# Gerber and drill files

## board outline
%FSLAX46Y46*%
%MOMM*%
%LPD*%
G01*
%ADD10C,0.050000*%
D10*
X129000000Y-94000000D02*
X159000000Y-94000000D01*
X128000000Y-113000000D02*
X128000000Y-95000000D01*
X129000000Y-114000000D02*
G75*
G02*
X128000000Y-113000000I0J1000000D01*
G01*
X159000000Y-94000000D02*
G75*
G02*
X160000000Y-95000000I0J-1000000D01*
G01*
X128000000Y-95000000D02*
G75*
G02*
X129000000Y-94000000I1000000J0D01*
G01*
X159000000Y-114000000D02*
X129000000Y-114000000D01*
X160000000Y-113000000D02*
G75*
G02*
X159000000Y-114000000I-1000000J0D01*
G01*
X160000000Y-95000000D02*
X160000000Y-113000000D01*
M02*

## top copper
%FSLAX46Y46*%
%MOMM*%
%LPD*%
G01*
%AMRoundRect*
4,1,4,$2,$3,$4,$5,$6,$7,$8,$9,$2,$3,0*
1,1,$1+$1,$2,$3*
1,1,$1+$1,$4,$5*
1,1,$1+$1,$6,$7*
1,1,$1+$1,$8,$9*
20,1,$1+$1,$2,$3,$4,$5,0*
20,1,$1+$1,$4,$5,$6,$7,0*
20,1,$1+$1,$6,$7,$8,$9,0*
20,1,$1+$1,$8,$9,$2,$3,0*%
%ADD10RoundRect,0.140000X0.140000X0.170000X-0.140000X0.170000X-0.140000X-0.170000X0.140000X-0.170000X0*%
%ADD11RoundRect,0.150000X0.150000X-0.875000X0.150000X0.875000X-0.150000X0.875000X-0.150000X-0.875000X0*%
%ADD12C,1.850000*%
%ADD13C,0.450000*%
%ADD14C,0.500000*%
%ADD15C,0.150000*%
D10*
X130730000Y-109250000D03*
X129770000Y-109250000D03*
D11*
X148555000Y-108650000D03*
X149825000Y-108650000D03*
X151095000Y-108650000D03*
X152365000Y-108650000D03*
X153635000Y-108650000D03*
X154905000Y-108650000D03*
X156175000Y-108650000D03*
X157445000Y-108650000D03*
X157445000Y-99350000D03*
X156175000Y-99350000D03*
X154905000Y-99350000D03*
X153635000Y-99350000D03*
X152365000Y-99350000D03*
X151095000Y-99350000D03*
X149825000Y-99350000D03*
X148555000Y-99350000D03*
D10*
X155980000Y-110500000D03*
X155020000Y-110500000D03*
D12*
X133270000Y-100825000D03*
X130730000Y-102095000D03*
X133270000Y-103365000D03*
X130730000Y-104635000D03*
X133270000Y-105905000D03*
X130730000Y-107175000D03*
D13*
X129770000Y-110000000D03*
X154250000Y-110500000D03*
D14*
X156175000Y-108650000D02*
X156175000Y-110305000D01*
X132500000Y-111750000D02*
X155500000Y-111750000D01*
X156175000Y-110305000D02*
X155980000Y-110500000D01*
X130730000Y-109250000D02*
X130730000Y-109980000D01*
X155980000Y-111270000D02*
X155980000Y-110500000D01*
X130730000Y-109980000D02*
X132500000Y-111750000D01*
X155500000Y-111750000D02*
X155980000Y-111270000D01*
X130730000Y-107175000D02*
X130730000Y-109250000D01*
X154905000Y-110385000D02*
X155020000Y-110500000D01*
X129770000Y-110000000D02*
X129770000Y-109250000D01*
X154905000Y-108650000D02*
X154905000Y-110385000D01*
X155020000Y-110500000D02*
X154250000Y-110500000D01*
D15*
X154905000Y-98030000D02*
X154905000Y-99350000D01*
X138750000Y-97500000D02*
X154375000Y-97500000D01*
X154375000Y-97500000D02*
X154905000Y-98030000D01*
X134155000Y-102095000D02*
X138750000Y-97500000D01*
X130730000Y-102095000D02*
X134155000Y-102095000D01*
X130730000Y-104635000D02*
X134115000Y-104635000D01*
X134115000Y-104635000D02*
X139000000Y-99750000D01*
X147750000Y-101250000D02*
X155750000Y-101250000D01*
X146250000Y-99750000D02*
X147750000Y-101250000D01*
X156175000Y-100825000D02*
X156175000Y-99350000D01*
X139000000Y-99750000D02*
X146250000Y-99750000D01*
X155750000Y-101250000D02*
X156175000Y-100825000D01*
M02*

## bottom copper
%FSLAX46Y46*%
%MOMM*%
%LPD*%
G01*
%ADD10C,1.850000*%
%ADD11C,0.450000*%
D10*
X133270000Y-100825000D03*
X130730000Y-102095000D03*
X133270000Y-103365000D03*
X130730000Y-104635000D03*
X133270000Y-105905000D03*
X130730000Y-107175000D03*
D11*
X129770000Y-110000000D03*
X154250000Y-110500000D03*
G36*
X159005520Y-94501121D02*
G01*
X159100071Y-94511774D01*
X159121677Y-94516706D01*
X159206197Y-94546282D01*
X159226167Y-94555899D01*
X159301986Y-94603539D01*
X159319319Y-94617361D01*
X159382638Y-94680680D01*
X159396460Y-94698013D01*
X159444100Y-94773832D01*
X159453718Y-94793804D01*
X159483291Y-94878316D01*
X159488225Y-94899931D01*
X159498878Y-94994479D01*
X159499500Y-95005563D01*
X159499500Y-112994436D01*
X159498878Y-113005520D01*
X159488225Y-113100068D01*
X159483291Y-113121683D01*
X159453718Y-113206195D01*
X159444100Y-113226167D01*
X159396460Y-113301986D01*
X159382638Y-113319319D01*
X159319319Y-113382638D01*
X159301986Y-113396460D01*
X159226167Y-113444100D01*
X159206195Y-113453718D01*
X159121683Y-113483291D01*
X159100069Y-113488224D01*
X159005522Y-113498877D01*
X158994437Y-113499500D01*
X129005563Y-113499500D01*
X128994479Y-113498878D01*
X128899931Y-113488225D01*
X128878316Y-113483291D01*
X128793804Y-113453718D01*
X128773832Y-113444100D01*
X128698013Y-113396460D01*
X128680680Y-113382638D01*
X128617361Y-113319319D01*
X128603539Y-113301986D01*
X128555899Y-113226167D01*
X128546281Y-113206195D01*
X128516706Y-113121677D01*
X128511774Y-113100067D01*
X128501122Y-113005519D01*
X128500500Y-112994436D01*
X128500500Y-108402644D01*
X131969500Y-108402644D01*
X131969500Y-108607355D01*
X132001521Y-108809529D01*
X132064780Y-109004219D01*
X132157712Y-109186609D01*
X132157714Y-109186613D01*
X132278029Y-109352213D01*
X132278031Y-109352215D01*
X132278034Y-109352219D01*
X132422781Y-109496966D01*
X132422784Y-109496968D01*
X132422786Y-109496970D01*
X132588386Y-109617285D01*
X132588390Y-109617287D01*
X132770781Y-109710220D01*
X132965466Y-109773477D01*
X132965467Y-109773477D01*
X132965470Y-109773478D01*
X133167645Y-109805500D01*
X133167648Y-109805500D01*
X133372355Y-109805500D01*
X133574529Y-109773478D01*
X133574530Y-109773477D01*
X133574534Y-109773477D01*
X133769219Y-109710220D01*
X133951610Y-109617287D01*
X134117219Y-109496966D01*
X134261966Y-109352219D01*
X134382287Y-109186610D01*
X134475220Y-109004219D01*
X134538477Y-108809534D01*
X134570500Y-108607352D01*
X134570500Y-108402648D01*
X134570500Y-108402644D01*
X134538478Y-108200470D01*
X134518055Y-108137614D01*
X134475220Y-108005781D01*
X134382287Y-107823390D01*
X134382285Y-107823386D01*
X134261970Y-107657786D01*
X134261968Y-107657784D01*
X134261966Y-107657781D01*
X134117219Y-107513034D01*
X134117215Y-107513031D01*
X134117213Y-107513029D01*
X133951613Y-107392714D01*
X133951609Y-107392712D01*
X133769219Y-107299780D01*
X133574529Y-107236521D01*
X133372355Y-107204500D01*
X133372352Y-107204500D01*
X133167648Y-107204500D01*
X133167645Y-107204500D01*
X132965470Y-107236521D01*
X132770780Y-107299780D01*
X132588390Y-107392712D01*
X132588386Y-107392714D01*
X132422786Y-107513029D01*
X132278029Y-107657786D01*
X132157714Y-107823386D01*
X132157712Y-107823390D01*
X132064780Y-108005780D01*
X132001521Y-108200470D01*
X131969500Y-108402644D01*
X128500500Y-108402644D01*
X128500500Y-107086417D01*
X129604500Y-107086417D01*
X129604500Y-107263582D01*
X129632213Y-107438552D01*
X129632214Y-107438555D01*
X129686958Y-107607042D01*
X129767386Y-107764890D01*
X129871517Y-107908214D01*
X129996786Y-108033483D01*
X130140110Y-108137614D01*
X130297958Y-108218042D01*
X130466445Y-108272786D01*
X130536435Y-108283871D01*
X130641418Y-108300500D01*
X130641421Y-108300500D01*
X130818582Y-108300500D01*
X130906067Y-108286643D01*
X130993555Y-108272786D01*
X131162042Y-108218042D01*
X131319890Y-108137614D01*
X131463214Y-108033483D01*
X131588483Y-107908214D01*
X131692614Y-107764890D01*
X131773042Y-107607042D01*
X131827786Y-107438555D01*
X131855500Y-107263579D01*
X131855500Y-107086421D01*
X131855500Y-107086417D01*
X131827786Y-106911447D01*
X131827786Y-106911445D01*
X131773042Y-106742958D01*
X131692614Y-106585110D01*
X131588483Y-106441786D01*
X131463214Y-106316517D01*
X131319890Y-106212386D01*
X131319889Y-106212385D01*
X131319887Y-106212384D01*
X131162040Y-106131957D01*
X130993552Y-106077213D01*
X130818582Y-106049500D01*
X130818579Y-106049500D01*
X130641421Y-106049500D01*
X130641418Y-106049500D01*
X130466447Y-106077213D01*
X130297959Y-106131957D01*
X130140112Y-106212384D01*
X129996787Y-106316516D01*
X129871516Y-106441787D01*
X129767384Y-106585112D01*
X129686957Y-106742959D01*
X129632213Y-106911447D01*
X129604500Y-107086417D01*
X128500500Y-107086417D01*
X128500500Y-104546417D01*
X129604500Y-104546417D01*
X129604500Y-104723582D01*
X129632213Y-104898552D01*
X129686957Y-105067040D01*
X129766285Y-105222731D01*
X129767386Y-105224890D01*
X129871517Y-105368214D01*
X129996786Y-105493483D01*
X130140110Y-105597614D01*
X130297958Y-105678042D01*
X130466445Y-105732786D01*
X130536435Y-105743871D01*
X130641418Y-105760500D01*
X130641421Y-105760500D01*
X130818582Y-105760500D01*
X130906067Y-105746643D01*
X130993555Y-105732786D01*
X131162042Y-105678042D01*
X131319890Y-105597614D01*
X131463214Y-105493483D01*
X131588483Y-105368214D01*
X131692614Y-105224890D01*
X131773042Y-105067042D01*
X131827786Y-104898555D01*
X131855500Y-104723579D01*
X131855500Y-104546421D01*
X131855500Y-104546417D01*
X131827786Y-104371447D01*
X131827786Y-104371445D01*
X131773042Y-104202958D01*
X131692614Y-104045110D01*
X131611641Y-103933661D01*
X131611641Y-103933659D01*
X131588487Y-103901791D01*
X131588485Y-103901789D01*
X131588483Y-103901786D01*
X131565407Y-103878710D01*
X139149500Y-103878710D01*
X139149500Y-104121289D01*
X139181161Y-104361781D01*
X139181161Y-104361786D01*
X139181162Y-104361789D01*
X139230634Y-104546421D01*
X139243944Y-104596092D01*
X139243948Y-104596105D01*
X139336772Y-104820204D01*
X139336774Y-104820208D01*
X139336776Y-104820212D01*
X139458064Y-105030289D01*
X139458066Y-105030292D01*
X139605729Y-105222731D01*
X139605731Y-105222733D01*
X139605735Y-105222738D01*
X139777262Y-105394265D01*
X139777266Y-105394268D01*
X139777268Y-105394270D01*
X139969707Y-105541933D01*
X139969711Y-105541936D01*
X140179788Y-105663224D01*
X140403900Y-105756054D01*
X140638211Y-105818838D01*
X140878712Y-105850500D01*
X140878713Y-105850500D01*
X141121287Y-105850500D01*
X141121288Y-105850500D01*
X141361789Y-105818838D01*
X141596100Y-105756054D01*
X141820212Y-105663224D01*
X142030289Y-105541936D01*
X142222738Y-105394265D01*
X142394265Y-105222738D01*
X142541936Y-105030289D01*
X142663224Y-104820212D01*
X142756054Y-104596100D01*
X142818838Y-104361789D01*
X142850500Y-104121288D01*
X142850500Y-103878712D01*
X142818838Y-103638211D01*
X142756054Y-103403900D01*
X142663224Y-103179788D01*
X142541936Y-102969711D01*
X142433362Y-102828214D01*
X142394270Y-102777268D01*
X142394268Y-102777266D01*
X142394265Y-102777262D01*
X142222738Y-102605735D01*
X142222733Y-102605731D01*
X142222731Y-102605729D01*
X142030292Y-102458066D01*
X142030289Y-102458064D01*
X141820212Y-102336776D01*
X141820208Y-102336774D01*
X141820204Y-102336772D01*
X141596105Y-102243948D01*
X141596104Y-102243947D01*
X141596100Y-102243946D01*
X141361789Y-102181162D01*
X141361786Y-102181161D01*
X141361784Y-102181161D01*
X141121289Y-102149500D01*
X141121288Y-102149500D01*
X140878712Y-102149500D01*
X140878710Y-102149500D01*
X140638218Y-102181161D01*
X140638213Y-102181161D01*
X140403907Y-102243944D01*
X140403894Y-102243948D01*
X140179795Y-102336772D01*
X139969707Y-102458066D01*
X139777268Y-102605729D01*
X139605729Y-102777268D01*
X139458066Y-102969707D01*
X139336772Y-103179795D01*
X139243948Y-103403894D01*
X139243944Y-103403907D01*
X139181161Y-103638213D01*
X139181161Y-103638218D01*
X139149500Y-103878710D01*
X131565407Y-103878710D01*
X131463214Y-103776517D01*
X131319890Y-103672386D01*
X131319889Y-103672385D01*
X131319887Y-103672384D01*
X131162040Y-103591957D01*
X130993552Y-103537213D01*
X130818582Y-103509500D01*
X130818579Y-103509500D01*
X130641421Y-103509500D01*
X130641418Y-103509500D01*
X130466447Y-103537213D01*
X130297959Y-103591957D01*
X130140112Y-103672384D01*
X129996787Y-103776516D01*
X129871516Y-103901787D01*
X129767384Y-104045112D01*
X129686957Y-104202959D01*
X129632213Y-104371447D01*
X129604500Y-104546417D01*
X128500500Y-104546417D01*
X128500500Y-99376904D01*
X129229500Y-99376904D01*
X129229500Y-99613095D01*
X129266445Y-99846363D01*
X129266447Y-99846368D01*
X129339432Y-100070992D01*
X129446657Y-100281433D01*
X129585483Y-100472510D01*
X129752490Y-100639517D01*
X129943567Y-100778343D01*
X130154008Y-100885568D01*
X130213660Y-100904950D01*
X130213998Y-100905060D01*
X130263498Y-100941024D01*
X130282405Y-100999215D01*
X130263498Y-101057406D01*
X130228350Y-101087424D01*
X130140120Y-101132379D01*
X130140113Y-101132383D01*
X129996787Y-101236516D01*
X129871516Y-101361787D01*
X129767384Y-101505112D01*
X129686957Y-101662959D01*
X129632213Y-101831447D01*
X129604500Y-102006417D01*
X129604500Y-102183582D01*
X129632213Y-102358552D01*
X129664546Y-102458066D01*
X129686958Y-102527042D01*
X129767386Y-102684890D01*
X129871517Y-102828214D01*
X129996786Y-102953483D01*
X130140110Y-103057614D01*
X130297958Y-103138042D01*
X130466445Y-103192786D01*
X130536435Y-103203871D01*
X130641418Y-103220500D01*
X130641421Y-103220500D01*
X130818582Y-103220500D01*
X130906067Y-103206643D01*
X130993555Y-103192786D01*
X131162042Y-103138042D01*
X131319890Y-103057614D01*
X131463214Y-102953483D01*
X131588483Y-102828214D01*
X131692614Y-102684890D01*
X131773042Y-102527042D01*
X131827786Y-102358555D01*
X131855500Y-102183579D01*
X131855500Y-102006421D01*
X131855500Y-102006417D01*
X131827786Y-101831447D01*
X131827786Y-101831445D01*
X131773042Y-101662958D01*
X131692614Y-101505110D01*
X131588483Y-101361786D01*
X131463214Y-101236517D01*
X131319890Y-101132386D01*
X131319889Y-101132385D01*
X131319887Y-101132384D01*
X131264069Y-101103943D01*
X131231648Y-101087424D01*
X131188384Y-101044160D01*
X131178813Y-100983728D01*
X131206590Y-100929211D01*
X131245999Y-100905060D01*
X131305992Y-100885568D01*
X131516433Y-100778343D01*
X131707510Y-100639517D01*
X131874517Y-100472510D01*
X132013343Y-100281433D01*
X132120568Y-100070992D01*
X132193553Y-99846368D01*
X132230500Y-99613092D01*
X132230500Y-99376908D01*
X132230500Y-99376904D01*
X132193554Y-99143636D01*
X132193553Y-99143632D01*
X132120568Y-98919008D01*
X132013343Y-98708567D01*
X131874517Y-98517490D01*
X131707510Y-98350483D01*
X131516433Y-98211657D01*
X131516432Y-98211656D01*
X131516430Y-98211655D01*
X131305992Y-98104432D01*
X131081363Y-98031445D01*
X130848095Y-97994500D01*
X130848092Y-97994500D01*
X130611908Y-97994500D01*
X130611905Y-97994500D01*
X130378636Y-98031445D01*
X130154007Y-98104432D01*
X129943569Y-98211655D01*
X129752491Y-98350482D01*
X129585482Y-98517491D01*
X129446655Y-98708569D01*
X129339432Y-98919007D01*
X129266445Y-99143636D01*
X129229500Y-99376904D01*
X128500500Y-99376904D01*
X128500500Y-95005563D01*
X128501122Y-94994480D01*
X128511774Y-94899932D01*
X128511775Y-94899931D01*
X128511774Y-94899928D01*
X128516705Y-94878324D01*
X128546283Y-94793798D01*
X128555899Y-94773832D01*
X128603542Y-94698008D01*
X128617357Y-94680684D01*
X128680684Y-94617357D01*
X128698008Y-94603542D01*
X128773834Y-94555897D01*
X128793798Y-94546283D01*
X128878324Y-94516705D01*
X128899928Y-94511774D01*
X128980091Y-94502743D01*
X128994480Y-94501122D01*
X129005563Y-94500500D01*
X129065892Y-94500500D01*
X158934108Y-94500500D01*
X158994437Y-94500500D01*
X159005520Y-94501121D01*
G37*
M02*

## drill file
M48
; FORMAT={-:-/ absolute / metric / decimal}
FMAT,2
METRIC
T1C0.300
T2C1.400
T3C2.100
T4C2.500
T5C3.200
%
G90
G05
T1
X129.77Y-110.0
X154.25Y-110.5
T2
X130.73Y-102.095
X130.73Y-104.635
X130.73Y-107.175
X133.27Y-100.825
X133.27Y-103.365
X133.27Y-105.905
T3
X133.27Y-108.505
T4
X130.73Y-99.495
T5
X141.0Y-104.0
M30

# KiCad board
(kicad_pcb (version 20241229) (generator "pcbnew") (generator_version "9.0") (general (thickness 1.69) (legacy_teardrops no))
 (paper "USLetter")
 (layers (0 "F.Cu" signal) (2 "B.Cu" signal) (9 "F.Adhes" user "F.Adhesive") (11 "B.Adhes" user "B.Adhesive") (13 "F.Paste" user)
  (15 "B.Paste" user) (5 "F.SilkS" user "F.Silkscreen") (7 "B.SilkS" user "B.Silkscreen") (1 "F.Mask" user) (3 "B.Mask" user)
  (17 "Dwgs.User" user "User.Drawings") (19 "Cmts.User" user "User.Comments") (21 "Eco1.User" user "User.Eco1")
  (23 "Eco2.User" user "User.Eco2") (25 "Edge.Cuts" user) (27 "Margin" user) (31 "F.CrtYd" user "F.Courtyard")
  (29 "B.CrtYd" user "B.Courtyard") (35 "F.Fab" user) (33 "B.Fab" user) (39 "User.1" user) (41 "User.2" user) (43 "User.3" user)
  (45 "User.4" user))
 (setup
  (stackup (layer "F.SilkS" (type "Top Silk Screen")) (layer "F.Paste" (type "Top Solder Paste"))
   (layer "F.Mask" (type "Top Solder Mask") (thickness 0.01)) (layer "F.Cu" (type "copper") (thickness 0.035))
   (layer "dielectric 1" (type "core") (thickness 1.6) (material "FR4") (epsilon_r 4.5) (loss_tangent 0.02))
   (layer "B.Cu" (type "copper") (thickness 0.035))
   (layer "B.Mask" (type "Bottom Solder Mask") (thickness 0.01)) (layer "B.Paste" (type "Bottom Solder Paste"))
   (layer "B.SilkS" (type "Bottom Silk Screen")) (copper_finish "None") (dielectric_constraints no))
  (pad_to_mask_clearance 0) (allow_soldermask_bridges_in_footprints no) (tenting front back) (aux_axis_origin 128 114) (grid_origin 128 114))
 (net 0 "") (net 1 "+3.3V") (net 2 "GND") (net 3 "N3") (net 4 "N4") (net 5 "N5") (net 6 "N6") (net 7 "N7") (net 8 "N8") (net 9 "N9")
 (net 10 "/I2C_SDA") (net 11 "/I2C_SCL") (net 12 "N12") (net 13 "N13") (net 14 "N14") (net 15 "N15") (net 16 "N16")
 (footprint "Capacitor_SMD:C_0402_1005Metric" (layer "F.Cu") (at 130.25 109.25 180)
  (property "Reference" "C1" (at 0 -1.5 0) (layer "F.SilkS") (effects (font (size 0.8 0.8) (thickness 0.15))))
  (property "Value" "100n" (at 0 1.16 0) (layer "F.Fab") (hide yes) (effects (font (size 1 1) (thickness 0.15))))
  (pad "1" smd roundrect (at -0.48 0 180) (size 0.56 0.62) (layers "F.Cu" "F.Mask" "F.Paste") (roundrect_rratio 0.25) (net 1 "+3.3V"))
  (pad "2" smd roundrect (at 0.48 0 180) (size 0.56 0.62) (layers "F.Cu" "F.Mask" "F.Paste") (roundrect_rratio 0.25) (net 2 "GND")))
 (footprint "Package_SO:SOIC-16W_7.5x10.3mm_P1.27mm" (layer "F.Cu") (at 153 104 90)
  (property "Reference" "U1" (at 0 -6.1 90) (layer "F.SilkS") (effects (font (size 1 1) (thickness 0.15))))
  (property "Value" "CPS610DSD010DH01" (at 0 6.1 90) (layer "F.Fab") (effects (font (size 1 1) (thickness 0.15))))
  (pad "1" smd roundrect (at -4.65 -4.445 90) (size 2.05 0.6) (layers "F.Cu" "F.Mask" "F.Paste") (roundrect_rratio 0.25) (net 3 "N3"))
  (pad "2" smd roundrect (at -4.65 -3.175 90) (size 2.05 0.6) (layers "F.Cu" "F.Mask" "F.Paste") (roundrect_rratio 0.25) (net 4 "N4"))
  (pad "3" smd roundrect (at -4.65 -1.905 90) (size 2.05 0.6) (layers "F.Cu" "F.Mask" "F.Paste") (roundrect_rratio 0.25) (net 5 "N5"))
  (pad "4" smd roundrect (at -4.65 -0.635 90) (size 2.05 0.6) (layers "F.Cu" "F.Mask" "F.Paste") (roundrect_rratio 0.25) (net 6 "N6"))
  (pad "5" smd roundrect (at -4.65 0.635 90) (size 2.05 0.6) (layers "F.Cu" "F.Mask" "F.Paste") (roundrect_rratio 0.25) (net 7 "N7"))
  (pad "6" smd roundrect (at -4.65 1.905 90) (size 2.05 0.6) (layers "F.Cu" "F.Mask" "F.Paste") (roundrect_rratio 0.25) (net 2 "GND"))
  (pad "7" smd roundrect (at -4.65 3.175 90) (size 2.05 0.6) (layers "F.Cu" "F.Mask" "F.Paste") (roundrect_rratio 0.25) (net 1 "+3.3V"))
  (pad "8" smd roundrect (at -4.65 4.445 90) (size 2.05 0.6) (layers "F.Cu" "F.Mask" "F.Paste") (roundrect_rratio 0.25) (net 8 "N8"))
  (pad "9" smd roundrect (at 4.65 4.445 90) (size 2.05 0.6) (layers "F.Cu" "F.Mask" "F.Paste") (roundrect_rratio 0.25) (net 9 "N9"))
  (pad "10" smd roundrect (at 4.65 3.175 90) (size 2.05 0.6) (layers "F.Cu" "F.Mask" "F.Paste") (roundrect_rratio 0.25) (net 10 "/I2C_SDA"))
  (pad "11" smd roundrect (at 4.65 1.905 90) (size 2.05 0.6) (layers "F.Cu" "F.Mask" "F.Paste") (roundrect_rratio 0.25) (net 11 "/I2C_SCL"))
  (pad "12" smd roundrect (at 4.65 0.635 90) (size 2.05 0.6) (layers "F.Cu" "F.Mask" "F.Paste") (roundrect_rratio 0.25) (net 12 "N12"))
  (pad "13" smd roundrect (at 4.65 -0.635 90) (size 2.05 0.6) (layers "F.Cu" "F.Mask" "F.Paste") (roundrect_rratio 0.25) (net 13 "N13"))
  (pad "14" smd roundrect (at 4.65 -1.905 90) (size 2.05 0.6) (layers "F.Cu" "F.Mask" "F.Paste") (roundrect_rratio 0.25) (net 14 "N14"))
  (pad "15" smd roundrect (at 4.65 -3.175 90) (size 2.05 0.6) (layers "F.Cu" "F.Mask" "F.Paste") (roundrect_rratio 0.25) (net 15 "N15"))
  (pad "16" smd roundrect (at 4.65 -4.445 90) (size 2.05 0.6) (layers "F.Cu" "F.Mask" "F.Paste") (roundrect_rratio 0.25) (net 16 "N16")))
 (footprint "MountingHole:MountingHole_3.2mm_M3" (layer "F.Cu") (at 141 104)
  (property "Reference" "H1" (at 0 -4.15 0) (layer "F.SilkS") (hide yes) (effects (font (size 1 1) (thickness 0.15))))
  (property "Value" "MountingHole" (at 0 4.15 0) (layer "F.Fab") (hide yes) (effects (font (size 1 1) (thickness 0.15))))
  (pad "" np_thru_hole circle (at 0 0) (size 3.2 3.2) (drill 3.2) (layers "*.Cu" "*.Mask")))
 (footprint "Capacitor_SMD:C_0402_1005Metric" (layer "F.Cu") (at 155.5 110.5 180)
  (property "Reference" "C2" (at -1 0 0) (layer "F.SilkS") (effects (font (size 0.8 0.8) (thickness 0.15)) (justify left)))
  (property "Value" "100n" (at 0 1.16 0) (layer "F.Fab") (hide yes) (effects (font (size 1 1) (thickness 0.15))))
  (pad "1" smd roundrect (at -0.48 0 180) (size 0.56 0.62) (layers "F.Cu" "F.Mask" "F.Paste") (roundrect_rratio 0.25) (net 1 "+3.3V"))
  (pad "2" smd roundrect (at 0.48 0 180) (size 0.56 0.62) (layers "F.Cu" "F.Mask" "F.Paste") (roundrect_rratio 0.25) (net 2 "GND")))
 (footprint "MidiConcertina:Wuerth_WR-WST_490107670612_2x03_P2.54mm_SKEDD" (layer "B.Cu") (at 132 104 180)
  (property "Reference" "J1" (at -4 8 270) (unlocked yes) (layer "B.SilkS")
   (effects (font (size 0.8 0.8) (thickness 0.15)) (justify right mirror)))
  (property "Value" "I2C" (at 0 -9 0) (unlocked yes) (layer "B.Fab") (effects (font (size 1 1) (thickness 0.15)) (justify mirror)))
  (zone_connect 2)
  (pad "" np_thru_hole circle (at -1.27 -4.505 180) (size 2.1 2.1) (drill 2.1) (layers "*.Cu" "*.Mask"))
  (pad "" np_thru_hole circle (at 1.27 4.505 180) (size 2.5 2.5) (drill 2.5) (layers "*.Cu" "*.Mask"))
  (pad "1" thru_hole circle (at -1.27 3.175 180) (size 1.85 1.85) (drill 1.4) (layers "*.Cu" "*.Mask") (remove_unused_layers no)
   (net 2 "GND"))
  (pad "2" thru_hole circle (at 1.27 1.905 180) (size 1.85 1.85) (drill 1.4) (layers "*.Cu" "*.Mask") (remove_unused_layers no)
   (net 11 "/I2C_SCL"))
  (pad "3" thru_hole circle (at -1.27 0.635 180) (size 1.85 1.85) (drill 1.4) (layers "*.Cu" "*.Mask") (remove_unused_layers no)
   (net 2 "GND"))
  (pad "4" thru_hole circle (at 1.27 -0.635 180) (size 1.85 1.85) (drill 1.4) (layers "*.Cu" "*.Mask") (remove_unused_layers no)
   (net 10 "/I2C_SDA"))
  (pad "5" thru_hole circle (at -1.27 -1.905 180) (size 1.85 1.85) (drill 1.4) (layers "*.Cu" "*.Mask") (remove_unused_layers no)
   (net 2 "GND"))
  (pad "6" thru_hole circle (at 1.27 -3.175 180) (size 1.85 1.85) (drill 1.4) (layers "*.Cu" "*.Mask") (remove_unused_layers no)
   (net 1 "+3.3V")))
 (gr_line (start 129 94) (end 159 94) (stroke (width 0.05) (type default)) (layer "Edge.Cuts"))
 (gr_line (start 128 113) (end 128 95) (stroke (width 0.05) (type default)) (layer "Edge.Cuts"))
 (gr_arc (start 129 114) (mid 128.292893 113.707107) (end 128 113) (stroke (width 0.05) (type default)) (layer "Edge.Cuts"))
 (gr_arc (start 159 94) (mid 159.707107 94.292893) (end 160 95) (stroke (width 0.05) (type default)) (layer "Edge.Cuts"))
 (gr_arc (start 128 95) (mid 128.292893 94.292893) (end 129 94) (stroke (width 0.05) (type default)) (layer "Edge.Cuts"))
 (gr_line (start 159 114) (end 129 114) (stroke (width 0.05) (type default)) (layer "Edge.Cuts"))
 (gr_arc (start 160 113) (mid 159.707107 113.707107) (end 159 114) (stroke (width 0.05) (type default)) (layer "Edge.Cuts"))
 (gr_line (start 160 95) (end 160 113) (stroke (width 0.05) (type default)) (layer "Edge.Cuts"))
 (segment (start 156.175 108.65) (end 156.175 110.305) (width 0.5) (layer "F.Cu") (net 1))
 (segment (start 132.5 111.75) (end 155.5 111.75) (width 0.5) (layer "F.Cu") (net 1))
 (segment (start 156.175 110.305) (end 155.98 110.5) (width 0.5) (layer "F.Cu") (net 1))
 (segment (start 130.73 109.25) (end 130.73 109.98) (width 0.5) (layer "F.Cu") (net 1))
 (segment (start 155.98 111.27) (end 155.98 110.5) (width 0.5) (layer "F.Cu") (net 1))
 (segment (start 130.73 109.98) (end 132.5 111.75) (width 0.5) (layer "F.Cu") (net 1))
 (segment (start 155.5 111.75) (end 155.98 111.27) (width 0.5) (layer "F.Cu") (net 1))
 (segment (start 130.73 107.175) (end 130.73 109.25) (width 0.5) (layer "F.Cu") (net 1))
 (segment (start 154.905 110.385) (end 155.02 110.5) (width 0.5) (layer "F.Cu") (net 2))
 (segment (start 129.77 110) (end 129.77 109.25) (width 0.5) (layer "F.Cu") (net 2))
 (segment (start 154.905 108.65) (end 154.905 110.385) (width 0.5) (layer "F.Cu") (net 2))
 (segment (start 155.02 110.5) (end 154.25 110.5) (width 0.5) (layer "F.Cu") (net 2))
 (via (at 129.77 110) (size 0.45) (drill 0.3) (layers "F.Cu" "B.Cu") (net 2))
 (via (at 154.25 110.5) (size 0.45) (drill 0.3) (layers "F.Cu" "B.Cu") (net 2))
 (segment (start 154.905 98.03) (end 154.905 99.35) (width 0.15) (layer "F.Cu") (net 11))
 (segment (start 138.75 97.5) (end 154.375 97.5) (width 0.15) (layer "F.Cu") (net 11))
 (segment (start 154.375 97.5) (end 154.905 98.03) (width 0.15) (layer "F.Cu") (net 11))
 (segment (start 134.155 102.095) (end 138.75 97.5) (width 0.15) (layer "F.Cu") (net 11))
 (segment (start 130.73 102.095) (end 134.155 102.095) (width 0.15) (layer "F.Cu") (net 11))
 (segment (start 130.73 104.635) (end 134.115 104.635) (width 0.15) (layer "F.Cu") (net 10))
 (segment (start 134.115 104.635) (end 139 99.75) (width 0.15) (layer "F.Cu") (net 10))
 (segment (start 147.75 101.25) (end 155.75 101.25) (width 0.15) (layer "F.Cu") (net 10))
 (segment (start 146.25 99.75) (end 147.75 101.25) (width 0.15) (layer "F.Cu") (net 10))
 (segment (start 156.175 100.825) (end 156.175 99.35) (width 0.15) (layer "F.Cu") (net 10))
 (segment (start 139 99.75) (end 146.25 99.75) (width 0.15) (layer "F.Cu") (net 10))
 (segment (start 155.75 101.25) (end 156.175 100.825) (width 0.15) (layer "F.Cu") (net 10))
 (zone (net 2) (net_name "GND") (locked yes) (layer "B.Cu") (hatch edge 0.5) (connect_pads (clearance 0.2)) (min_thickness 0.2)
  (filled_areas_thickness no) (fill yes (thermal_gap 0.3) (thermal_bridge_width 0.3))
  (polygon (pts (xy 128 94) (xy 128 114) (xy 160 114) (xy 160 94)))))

